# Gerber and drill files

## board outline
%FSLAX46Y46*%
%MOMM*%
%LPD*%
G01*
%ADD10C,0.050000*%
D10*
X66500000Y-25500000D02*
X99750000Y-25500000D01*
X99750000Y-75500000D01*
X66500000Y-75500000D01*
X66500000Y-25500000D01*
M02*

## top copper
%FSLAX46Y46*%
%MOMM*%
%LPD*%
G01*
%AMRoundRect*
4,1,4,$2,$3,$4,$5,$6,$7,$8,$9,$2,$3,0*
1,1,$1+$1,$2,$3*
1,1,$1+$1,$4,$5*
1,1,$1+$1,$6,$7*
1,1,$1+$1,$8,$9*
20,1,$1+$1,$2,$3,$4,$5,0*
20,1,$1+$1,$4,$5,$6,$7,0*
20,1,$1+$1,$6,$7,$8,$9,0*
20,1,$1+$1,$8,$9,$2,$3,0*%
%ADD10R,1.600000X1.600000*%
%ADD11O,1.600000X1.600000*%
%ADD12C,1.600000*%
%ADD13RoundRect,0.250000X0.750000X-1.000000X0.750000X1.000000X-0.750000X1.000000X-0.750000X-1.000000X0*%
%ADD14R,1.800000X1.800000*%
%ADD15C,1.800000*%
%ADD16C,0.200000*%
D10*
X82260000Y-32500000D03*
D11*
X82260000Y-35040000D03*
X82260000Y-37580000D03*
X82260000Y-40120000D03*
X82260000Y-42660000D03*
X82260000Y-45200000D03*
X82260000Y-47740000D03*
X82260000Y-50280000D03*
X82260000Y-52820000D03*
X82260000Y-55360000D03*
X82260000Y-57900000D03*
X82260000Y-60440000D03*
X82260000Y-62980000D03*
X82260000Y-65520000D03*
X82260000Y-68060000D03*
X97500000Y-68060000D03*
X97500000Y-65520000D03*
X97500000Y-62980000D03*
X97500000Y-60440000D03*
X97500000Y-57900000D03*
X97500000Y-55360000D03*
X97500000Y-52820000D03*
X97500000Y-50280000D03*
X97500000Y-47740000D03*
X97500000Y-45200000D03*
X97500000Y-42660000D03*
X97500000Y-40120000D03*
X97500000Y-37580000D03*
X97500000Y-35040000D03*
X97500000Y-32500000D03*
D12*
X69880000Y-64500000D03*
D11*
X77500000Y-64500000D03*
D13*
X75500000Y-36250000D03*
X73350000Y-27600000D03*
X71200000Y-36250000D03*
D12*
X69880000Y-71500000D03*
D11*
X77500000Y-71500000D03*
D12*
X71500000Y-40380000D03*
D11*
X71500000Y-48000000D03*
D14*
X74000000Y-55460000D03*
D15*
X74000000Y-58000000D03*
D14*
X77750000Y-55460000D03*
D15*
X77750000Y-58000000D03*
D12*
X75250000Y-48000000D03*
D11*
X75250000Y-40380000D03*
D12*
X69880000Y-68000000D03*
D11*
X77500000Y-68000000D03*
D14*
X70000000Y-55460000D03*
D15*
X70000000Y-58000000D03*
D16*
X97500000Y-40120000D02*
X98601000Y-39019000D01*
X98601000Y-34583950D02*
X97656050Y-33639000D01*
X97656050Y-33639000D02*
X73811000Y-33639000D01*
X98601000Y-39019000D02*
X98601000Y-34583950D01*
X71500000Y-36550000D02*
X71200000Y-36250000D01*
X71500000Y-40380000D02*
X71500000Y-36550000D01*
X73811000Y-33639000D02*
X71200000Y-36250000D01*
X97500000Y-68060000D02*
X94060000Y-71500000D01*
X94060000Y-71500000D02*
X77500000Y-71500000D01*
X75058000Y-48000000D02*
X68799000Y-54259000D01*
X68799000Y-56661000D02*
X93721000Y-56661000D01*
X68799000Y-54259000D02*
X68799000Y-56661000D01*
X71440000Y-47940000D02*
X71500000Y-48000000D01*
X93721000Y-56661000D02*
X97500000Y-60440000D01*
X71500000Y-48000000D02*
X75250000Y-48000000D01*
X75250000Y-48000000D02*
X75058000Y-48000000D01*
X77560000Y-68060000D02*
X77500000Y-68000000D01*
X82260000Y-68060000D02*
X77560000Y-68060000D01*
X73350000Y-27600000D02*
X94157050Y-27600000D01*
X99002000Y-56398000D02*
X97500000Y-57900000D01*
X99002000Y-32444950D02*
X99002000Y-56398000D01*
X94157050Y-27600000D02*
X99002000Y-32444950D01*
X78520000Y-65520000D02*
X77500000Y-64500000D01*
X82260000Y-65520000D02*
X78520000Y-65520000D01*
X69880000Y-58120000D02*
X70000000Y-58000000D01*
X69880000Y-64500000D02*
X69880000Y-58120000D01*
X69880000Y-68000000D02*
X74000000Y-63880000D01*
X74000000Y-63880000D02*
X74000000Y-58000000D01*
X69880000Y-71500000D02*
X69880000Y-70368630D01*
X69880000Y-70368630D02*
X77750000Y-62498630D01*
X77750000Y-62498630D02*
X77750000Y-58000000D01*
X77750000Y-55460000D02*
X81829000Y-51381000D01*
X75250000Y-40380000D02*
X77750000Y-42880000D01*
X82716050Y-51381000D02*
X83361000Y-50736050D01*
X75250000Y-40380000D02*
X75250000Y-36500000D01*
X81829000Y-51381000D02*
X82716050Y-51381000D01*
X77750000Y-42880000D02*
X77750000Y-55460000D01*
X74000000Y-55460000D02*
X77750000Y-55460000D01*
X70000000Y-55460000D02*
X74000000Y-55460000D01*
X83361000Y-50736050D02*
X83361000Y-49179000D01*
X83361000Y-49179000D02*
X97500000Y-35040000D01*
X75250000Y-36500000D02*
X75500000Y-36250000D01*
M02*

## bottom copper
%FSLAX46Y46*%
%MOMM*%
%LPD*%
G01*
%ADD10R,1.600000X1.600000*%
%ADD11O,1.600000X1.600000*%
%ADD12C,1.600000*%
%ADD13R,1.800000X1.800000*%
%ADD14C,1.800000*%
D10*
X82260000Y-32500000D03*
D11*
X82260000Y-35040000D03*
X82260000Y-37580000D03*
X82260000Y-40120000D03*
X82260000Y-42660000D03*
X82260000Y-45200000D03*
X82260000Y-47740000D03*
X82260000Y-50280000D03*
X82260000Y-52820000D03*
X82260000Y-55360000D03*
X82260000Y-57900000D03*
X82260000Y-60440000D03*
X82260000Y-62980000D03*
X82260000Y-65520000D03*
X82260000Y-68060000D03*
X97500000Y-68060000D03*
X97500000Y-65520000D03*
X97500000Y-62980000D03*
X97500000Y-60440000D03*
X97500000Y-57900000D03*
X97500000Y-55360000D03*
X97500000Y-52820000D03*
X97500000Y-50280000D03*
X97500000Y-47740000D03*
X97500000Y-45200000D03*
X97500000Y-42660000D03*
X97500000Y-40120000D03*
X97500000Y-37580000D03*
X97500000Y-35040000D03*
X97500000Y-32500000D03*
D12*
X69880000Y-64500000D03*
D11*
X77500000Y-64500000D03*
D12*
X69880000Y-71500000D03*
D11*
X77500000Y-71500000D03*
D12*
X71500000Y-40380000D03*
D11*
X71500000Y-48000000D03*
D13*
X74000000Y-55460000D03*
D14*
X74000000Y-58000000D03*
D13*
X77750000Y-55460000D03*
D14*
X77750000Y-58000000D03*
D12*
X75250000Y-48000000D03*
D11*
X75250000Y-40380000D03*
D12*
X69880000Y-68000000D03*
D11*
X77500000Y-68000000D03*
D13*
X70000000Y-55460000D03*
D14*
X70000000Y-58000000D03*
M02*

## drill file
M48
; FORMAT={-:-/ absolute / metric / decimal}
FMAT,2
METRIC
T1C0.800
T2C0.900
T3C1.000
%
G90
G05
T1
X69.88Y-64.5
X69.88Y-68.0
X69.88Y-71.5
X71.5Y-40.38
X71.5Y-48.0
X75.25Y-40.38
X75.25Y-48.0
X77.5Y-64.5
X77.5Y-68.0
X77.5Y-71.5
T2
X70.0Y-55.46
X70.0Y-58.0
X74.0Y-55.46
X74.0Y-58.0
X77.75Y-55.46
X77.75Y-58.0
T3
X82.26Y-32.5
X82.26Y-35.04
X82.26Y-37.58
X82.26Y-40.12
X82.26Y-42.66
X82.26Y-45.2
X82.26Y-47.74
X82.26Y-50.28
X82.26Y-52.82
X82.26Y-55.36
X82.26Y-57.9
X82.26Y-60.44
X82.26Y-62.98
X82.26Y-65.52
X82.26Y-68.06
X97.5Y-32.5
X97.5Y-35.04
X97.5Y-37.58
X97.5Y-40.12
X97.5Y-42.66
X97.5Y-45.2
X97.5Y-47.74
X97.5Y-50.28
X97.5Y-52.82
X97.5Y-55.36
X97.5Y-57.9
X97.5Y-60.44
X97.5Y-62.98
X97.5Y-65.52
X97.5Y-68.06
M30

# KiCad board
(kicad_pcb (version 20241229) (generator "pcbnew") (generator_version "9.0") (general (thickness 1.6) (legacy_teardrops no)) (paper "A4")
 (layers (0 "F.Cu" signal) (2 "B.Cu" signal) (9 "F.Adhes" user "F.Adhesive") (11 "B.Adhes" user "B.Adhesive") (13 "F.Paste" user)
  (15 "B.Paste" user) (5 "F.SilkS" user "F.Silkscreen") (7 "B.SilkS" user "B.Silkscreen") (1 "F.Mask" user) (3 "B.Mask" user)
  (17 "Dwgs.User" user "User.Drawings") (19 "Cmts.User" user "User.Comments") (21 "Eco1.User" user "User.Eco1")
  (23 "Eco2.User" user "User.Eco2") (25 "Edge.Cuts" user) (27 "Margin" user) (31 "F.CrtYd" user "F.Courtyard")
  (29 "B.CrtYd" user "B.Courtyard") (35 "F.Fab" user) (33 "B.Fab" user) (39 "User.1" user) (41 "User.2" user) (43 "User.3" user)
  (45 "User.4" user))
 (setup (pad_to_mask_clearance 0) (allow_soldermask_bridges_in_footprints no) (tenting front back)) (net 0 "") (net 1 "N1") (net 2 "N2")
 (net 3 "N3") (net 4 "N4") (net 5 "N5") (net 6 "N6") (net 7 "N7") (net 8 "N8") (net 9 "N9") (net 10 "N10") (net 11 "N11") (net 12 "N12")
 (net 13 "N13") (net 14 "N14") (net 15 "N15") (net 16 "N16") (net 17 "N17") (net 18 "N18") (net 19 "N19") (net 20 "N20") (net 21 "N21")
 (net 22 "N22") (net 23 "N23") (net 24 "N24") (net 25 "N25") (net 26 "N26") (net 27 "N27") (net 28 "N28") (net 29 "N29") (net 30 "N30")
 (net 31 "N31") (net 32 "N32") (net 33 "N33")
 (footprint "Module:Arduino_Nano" (layer "F.Cu") (at 82.26 32.5)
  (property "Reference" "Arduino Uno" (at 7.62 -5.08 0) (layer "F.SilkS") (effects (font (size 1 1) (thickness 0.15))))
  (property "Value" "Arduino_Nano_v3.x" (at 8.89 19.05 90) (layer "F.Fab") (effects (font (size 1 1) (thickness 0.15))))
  (pad "1" thru_hole rect (at 0 0) (size 1.6 1.6) (drill 1) (layers "*.Cu" "*.Mask") (remove_unused_layers no) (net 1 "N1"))
  (pad "2" thru_hole oval (at 0 2.54) (size 1.6 1.6) (drill 1) (layers "*.Cu" "*.Mask") (remove_unused_layers no) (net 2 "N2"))
  (pad "3" thru_hole oval (at 0 5.08) (size 1.6 1.6) (drill 1) (layers "*.Cu" "*.Mask") (remove_unused_layers no) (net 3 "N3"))
  (pad "4" thru_hole oval (at 0 7.62) (size 1.6 1.6) (drill 1) (layers "*.Cu" "*.Mask") (remove_unused_layers no) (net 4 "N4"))
  (pad "5" thru_hole oval (at 0 10.16) (size 1.6 1.6) (drill 1) (layers "*.Cu" "*.Mask") (remove_unused_layers no) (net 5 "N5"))
  (pad "6" thru_hole oval (at 0 12.7) (size 1.6 1.6) (drill 1) (layers "*.Cu" "*.Mask") (remove_unused_layers no) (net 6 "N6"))
  (pad "7" thru_hole oval (at 0 15.24) (size 1.6 1.6) (drill 1) (layers "*.Cu" "*.Mask") (remove_unused_layers no) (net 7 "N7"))
  (pad "8" thru_hole oval (at 0 17.78) (size 1.6 1.6) (drill 1) (layers "*.Cu" "*.Mask") (remove_unused_layers no) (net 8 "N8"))
  (pad "9" thru_hole oval (at 0 20.32) (size 1.6 1.6) (drill 1) (layers "*.Cu" "*.Mask") (remove_unused_layers no) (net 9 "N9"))
  (pad "10" thru_hole oval (at 0 22.86) (size 1.6 1.6) (drill 1) (layers "*.Cu" "*.Mask") (remove_unused_layers no) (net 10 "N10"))
  (pad "11" thru_hole oval (at 0 25.4) (size 1.6 1.6) (drill 1) (layers "*.Cu" "*.Mask") (remove_unused_layers no) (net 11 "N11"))
  (pad "12" thru_hole oval (at 0 27.94) (size 1.6 1.6) (drill 1) (layers "*.Cu" "*.Mask") (remove_unused_layers no) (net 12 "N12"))
  (pad "13" thru_hole oval (at 0 30.48) (size 1.6 1.6) (drill 1) (layers "*.Cu" "*.Mask") (remove_unused_layers no) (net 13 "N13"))
  (pad "14" thru_hole oval (at 0 33.02) (size 1.6 1.6) (drill 1) (layers "*.Cu" "*.Mask") (remove_unused_layers no) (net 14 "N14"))
  (pad "15" thru_hole oval (at 0 35.56) (size 1.6 1.6) (drill 1) (layers "*.Cu" "*.Mask") (remove_unused_layers no) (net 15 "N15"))
  (pad "16" thru_hole oval (at 15.24 35.56) (size 1.6 1.6) (drill 1) (layers "*.Cu" "*.Mask") (remove_unused_layers no) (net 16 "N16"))
  (pad "17" thru_hole oval (at 15.24 33.02) (size 1.6 1.6) (drill 1) (layers "*.Cu" "*.Mask") (remove_unused_layers no) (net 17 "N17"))
  (pad "18" thru_hole oval (at 15.24 30.48) (size 1.6 1.6) (drill 1) (layers "*.Cu" "*.Mask") (remove_unused_layers no) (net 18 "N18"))
  (pad "19" thru_hole oval (at 15.24 27.94) (size 1.6 1.6) (drill 1) (layers "*.Cu" "*.Mask") (remove_unused_layers no) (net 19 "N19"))
  (pad "20" thru_hole oval (at 15.24 25.4) (size 1.6 1.6) (drill 1) (layers "*.Cu" "*.Mask") (remove_unused_layers no) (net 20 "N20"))
  (pad "21" thru_hole oval (at 15.24 22.86) (size 1.6 1.6) (drill 1) (layers "*.Cu" "*.Mask") (remove_unused_layers no) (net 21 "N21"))
  (pad "22" thru_hole oval (at 15.24 20.32) (size 1.6 1.6) (drill 1) (layers "*.Cu" "*.Mask") (remove_unused_layers no) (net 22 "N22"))
  (pad "23" thru_hole oval (at 15.24 17.78) (size 1.6 1.6) (drill 1) (layers "*.Cu" "*.Mask") (remove_unused_layers no) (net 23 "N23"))
  (pad "24" thru_hole oval (at 15.24 15.24) (size 1.6 1.6) (drill 1) (layers "*.Cu" "*.Mask") (remove_unused_layers no) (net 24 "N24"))
  (pad "25" thru_hole oval (at 15.24 12.7) (size 1.6 1.6) (drill 1) (layers "*.Cu" "*.Mask") (remove_unused_layers no) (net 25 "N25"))
  (pad "26" thru_hole oval (at 15.24 10.16) (size 1.6 1.6) (drill 1) (layers "*.Cu" "*.Mask") (remove_unused_layers no) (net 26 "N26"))
  (pad "27" thru_hole oval (at 15.24 7.62) (size 1.6 1.6) (drill 1) (layers "*.Cu" "*.Mask") (remove_unused_layers no) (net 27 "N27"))
  (pad "28" thru_hole oval (at 15.24 5.08) (size 1.6 1.6) (drill 1) (layers "*.Cu" "*.Mask") (remove_unused_layers no) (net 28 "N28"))
  (pad "29" thru_hole oval (at 15.24 2.54) (size 1.6 1.6) (drill 1) (layers "*.Cu" "*.Mask") (remove_unused_layers no) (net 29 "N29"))
  (pad "30" thru_hole oval (at 15.24 0) (size 1.6 1.6) (drill 1) (layers "*.Cu" "*.Mask") (remove_unused_layers no) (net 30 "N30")))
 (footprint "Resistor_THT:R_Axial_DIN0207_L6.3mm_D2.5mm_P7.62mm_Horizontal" (layer "F.Cu") (at 69.88 64.5)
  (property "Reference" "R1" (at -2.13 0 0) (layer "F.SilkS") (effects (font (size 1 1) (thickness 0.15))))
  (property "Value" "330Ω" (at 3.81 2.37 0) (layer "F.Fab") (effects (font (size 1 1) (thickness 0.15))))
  (pad "1" thru_hole circle (at 0 0) (size 1.6 1.6) (drill 0.8) (layers "*.Cu" "*.Mask") (remove_unused_layers no) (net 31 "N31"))
  (pad "2" thru_hole oval (at 7.62 0) (size 1.6 1.6) (drill 0.8) (layers "*.Cu" "*.Mask") (remove_unused_layers no) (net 14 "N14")))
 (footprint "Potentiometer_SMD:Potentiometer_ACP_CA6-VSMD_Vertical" (layer "F.Cu") (at 73.35 31.925 90)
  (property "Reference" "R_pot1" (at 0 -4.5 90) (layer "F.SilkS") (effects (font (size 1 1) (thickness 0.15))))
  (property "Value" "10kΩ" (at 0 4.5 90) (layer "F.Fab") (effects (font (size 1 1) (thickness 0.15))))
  (pad "1" smd roundrect (at -4.325 2.15 90) (size 2.5 2) (layers "F.Cu" "F.Mask" "F.Paste") (roundrect_rratio 0.125) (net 29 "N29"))
  (pad "2" smd roundrect (at 4.325 0 90) (size 2.5 2) (layers "F.Cu" "F.Mask" "F.Paste") (roundrect_rratio 0.125) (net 20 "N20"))
  (pad "3" smd roundrect (at -4.325 -2.15 90) (size 2.5 2) (layers "F.Cu" "F.Mask" "F.Paste") (roundrect_rratio 0.125) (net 27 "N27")))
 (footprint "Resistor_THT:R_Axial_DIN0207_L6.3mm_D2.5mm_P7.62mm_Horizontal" (layer "F.Cu") (at 69.88 71.5)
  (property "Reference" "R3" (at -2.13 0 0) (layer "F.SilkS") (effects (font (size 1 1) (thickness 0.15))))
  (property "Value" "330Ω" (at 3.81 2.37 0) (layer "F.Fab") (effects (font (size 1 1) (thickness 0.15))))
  (pad "1" thru_hole circle (at 0 0) (size 1.6 1.6) (drill 0.8) (layers "*.Cu" "*.Mask") (remove_unused_layers no) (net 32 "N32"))
  (pad "2" thru_hole oval (at 7.62 0) (size 1.6 1.6) (drill 0.8) (layers "*.Cu" "*.Mask") (remove_unused_layers no) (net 16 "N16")))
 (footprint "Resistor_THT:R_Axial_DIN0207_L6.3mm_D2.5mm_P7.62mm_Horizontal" (layer "F.Cu") (at 71.5 40.38 -90)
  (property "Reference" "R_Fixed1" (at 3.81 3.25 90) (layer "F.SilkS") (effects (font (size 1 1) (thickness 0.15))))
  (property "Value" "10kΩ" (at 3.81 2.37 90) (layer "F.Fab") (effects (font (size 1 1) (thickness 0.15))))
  (pad "1" thru_hole circle (at 0 0 270) (size 1.6 1.6) (drill 0.8) (layers "*.Cu" "*.Mask") (remove_unused_layers no) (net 27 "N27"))
  (pad "2" thru_hole oval (at 7.62 0 270) (size 1.6 1.6) (drill 0.8) (layers "*.Cu" "*.Mask") (remove_unused_layers no) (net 19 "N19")))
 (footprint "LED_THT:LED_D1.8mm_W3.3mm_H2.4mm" (layer "F.Cu") (at 74 55.46 -90)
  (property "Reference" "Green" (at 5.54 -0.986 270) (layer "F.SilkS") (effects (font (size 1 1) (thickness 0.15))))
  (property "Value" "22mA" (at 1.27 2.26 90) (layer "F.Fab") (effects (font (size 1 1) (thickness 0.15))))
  (pad "1" thru_hole rect (at 0 0 270) (size 1.8 1.8) (drill 0.9) (layers "*.Cu" "*.Mask") (remove_unused_layers no) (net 29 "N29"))
  (pad "2" thru_hole circle (at 2.54 0 270) (size 1.8 1.8) (drill 0.9) (layers "*.Cu" "*.Mask") (remove_unused_layers no) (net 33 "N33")))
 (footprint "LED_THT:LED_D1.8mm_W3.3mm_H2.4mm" (layer "F.Cu") (at 77.75 55.46 -90)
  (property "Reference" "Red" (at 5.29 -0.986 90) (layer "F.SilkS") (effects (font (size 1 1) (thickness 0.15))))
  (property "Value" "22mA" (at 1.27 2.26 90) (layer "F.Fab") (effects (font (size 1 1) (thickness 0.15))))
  (pad "1" thru_hole rect (at 0 0 270) (size 1.8 1.8) (drill 0.9) (layers "*.Cu" "*.Mask") (remove_unused_layers no) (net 29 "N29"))
  (pad "2" thru_hole circle (at 2.54 0 270) (size 1.8 1.8) (drill 0.9) (layers "*.Cu" "*.Mask") (remove_unused_layers no) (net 32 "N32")))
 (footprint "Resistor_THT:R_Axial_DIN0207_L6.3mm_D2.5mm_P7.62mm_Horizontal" (layer "F.Cu") (at 75.25 48 90)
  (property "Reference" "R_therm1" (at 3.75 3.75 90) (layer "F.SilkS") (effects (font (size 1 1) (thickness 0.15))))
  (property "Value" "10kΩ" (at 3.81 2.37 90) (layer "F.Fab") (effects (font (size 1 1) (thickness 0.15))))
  (pad "1" thru_hole circle (at 0 0 90) (size 1.6 1.6) (drill 0.8) (layers "*.Cu" "*.Mask") (remove_unused_layers no) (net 19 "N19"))
  (pad "2" thru_hole oval (at 7.62 0 90) (size 1.6 1.6) (drill 0.8) (layers "*.Cu" "*.Mask") (remove_unused_layers no) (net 29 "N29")))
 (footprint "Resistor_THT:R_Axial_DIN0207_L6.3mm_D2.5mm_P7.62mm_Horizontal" (layer "F.Cu") (at 69.88 68)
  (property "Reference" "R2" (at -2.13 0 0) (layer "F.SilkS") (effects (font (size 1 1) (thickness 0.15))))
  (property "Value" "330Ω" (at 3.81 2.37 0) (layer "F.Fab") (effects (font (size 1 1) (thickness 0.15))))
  (pad "1" thru_hole circle (at 0 0) (size 1.6 1.6) (drill 0.8) (layers "*.Cu" "*.Mask") (remove_unused_layers no) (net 33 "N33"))
  (pad "2" thru_hole oval (at 7.62 0) (size 1.6 1.6) (drill 0.8) (layers "*.Cu" "*.Mask") (remove_unused_layers no) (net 15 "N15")))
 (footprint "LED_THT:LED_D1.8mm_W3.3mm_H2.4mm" (layer "F.Cu") (at 70 55.46 -90)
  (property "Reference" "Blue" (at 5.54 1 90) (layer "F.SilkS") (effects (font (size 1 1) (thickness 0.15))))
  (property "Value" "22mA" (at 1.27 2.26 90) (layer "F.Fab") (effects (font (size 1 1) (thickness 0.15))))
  (pad "1" thru_hole rect (at 0 0 270) (size 1.8 1.8) (drill 0.9) (layers "*.Cu" "*.Mask") (remove_unused_layers no) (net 29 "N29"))
  (pad "2" thru_hole circle (at 2.54 0 270) (size 1.8 1.8) (drill 0.9) (layers "*.Cu" "*.Mask") (remove_unused_layers no) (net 31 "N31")))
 (gr_rect (start 66.5 25.5) (end 99.75 75.5) (stroke (width 0.05) (type default)) (fill no) (layer "Edge.Cuts"))
 (segment (start 97.5 40.12) (end 98.601 39.019) (width 0.2) (layer "F.Cu") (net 27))
 (segment (start 98.601 34.58395) (end 97.65605 33.639) (width 0.2) (layer "F.Cu") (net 27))
 (segment (start 97.65605 33.639) (end 73.811 33.639) (width 0.2) (layer "F.Cu") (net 27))
 (segment (start 98.601 39.019) (end 98.601 34.58395) (width 0.2) (layer "F.Cu") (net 27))
 (segment (start 71.5 36.55) (end 71.2 36.25) (width 0.2) (layer "F.Cu") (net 27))
 (segment (start 71.5 40.38) (end 71.5 36.55) (width 0.2) (layer "F.Cu") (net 27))
 (segment (start 73.811 33.639) (end 71.2 36.25) (width 0.2) (layer "F.Cu") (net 27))
 (segment (start 97.5 68.06) (end 94.06 71.5) (width 0.2) (layer "F.Cu") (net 16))
 (segment (start 94.06 71.5) (end 77.5 71.5) (width 0.2) (layer "F.Cu") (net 16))
 (segment (start 75.058 48) (end 68.799 54.259) (width 0.2) (layer "F.Cu") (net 19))
 (segment (start 68.799 56.661) (end 93.721 56.661) (width 0.2) (layer "F.Cu") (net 19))
 (segment (start 68.799 54.259) (end 68.799 56.661) (width 0.2) (layer "F.Cu") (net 19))
 (segment (start 71.44 47.94) (end 71.5 48) (width 0.2) (layer "F.Cu") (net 19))
 (segment (start 93.721 56.661) (end 97.5 60.44) (width 0.2) (layer "F.Cu") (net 19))
 (segment (start 71.5 48) (end 75.25 48) (width 0.2) (layer "F.Cu") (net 19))
 (segment (start 75.25 48) (end 75.058 48) (width 0.2) (layer "F.Cu") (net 19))
 (segment (start 77.56 68.06) (end 77.5 68) (width 0.2) (layer "F.Cu") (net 15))
 (segment (start 82.26 68.06) (end 77.56 68.06) (width 0.2) (layer "F.Cu") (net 15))
 (segment (start 73.35 27.6) (end 94.15705 27.6) (width 0.2) (layer "F.Cu") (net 20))
 (segment (start 99.002 56.398) (end 97.5 57.9) (width 0.2) (layer "F.Cu") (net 20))
 (segment (start 99.002 32.44495) (end 99.002 56.398) (width 0.2) (layer "F.Cu") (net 20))
 (segment (start 94.15705 27.6) (end 99.002 32.44495) (width 0.2) (layer "F.Cu") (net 20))
 (segment (start 78.52 65.52) (end 77.5 64.5) (width 0.2) (layer "F.Cu") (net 14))
 (segment (start 82.26 65.52) (end 78.52 65.52) (width 0.2) (layer "F.Cu") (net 14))
 (segment (start 69.88 58.12) (end 70 58) (width 0.2) (layer "F.Cu") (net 31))
 (segment (start 69.88 64.5) (end 69.88 58.12) (width 0.2) (layer "F.Cu") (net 31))
 (segment (start 69.88 68) (end 74 63.88) (width 0.2) (layer "F.Cu") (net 33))
 (segment (start 74 63.88) (end 74 58) (width 0.2) (layer "F.Cu") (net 33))
 (segment (start 69.88 71.5) (end 69.88 70.36863) (width 0.2) (layer "F.Cu") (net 32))
 (segment (start 69.88 70.36863) (end 77.75 62.49863) (width 0.2) (layer "F.Cu") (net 32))
 (segment (start 77.75 62.49863) (end 77.75 58) (width 0.2) (layer "F.Cu") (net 32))
 (segment (start 77.75 55.46) (end 81.829 51.381) (width 0.2) (layer "F.Cu") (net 29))
 (segment (start 75.25 40.38) (end 77.75 42.88) (width 0.2) (layer "F.Cu") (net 29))
 (segment (start 82.71605 51.381) (end 83.361 50.73605) (width 0.2) (layer "F.Cu") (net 29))
 (segment (start 75.25 40.38) (end 75.25 36.5) (width 0.2) (layer "F.Cu") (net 29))
 (segment (start 81.829 51.381) (end 82.71605 51.381) (width 0.2) (layer "F.Cu") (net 29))
 (segment (start 77.75 42.88) (end 77.75 55.46) (width 0.2) (layer "F.Cu") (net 29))
 (segment (start 74 55.46) (end 77.75 55.46) (width 0.2) (layer "F.Cu") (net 29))
 (segment (start 70 55.46) (end 74 55.46) (width 0.2) (layer "F.Cu") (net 29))
 (segment (start 83.361 50.73605) (end 83.361 49.179) (width 0.2) (layer "F.Cu") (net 29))
 (segment (start 83.361 49.179) (end 97.5 35.04) (width 0.2) (layer "F.Cu") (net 29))
 (segment (start 75.25 36.5) (end 75.5 36.25) (width 0.2) (layer "F.Cu") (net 29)))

